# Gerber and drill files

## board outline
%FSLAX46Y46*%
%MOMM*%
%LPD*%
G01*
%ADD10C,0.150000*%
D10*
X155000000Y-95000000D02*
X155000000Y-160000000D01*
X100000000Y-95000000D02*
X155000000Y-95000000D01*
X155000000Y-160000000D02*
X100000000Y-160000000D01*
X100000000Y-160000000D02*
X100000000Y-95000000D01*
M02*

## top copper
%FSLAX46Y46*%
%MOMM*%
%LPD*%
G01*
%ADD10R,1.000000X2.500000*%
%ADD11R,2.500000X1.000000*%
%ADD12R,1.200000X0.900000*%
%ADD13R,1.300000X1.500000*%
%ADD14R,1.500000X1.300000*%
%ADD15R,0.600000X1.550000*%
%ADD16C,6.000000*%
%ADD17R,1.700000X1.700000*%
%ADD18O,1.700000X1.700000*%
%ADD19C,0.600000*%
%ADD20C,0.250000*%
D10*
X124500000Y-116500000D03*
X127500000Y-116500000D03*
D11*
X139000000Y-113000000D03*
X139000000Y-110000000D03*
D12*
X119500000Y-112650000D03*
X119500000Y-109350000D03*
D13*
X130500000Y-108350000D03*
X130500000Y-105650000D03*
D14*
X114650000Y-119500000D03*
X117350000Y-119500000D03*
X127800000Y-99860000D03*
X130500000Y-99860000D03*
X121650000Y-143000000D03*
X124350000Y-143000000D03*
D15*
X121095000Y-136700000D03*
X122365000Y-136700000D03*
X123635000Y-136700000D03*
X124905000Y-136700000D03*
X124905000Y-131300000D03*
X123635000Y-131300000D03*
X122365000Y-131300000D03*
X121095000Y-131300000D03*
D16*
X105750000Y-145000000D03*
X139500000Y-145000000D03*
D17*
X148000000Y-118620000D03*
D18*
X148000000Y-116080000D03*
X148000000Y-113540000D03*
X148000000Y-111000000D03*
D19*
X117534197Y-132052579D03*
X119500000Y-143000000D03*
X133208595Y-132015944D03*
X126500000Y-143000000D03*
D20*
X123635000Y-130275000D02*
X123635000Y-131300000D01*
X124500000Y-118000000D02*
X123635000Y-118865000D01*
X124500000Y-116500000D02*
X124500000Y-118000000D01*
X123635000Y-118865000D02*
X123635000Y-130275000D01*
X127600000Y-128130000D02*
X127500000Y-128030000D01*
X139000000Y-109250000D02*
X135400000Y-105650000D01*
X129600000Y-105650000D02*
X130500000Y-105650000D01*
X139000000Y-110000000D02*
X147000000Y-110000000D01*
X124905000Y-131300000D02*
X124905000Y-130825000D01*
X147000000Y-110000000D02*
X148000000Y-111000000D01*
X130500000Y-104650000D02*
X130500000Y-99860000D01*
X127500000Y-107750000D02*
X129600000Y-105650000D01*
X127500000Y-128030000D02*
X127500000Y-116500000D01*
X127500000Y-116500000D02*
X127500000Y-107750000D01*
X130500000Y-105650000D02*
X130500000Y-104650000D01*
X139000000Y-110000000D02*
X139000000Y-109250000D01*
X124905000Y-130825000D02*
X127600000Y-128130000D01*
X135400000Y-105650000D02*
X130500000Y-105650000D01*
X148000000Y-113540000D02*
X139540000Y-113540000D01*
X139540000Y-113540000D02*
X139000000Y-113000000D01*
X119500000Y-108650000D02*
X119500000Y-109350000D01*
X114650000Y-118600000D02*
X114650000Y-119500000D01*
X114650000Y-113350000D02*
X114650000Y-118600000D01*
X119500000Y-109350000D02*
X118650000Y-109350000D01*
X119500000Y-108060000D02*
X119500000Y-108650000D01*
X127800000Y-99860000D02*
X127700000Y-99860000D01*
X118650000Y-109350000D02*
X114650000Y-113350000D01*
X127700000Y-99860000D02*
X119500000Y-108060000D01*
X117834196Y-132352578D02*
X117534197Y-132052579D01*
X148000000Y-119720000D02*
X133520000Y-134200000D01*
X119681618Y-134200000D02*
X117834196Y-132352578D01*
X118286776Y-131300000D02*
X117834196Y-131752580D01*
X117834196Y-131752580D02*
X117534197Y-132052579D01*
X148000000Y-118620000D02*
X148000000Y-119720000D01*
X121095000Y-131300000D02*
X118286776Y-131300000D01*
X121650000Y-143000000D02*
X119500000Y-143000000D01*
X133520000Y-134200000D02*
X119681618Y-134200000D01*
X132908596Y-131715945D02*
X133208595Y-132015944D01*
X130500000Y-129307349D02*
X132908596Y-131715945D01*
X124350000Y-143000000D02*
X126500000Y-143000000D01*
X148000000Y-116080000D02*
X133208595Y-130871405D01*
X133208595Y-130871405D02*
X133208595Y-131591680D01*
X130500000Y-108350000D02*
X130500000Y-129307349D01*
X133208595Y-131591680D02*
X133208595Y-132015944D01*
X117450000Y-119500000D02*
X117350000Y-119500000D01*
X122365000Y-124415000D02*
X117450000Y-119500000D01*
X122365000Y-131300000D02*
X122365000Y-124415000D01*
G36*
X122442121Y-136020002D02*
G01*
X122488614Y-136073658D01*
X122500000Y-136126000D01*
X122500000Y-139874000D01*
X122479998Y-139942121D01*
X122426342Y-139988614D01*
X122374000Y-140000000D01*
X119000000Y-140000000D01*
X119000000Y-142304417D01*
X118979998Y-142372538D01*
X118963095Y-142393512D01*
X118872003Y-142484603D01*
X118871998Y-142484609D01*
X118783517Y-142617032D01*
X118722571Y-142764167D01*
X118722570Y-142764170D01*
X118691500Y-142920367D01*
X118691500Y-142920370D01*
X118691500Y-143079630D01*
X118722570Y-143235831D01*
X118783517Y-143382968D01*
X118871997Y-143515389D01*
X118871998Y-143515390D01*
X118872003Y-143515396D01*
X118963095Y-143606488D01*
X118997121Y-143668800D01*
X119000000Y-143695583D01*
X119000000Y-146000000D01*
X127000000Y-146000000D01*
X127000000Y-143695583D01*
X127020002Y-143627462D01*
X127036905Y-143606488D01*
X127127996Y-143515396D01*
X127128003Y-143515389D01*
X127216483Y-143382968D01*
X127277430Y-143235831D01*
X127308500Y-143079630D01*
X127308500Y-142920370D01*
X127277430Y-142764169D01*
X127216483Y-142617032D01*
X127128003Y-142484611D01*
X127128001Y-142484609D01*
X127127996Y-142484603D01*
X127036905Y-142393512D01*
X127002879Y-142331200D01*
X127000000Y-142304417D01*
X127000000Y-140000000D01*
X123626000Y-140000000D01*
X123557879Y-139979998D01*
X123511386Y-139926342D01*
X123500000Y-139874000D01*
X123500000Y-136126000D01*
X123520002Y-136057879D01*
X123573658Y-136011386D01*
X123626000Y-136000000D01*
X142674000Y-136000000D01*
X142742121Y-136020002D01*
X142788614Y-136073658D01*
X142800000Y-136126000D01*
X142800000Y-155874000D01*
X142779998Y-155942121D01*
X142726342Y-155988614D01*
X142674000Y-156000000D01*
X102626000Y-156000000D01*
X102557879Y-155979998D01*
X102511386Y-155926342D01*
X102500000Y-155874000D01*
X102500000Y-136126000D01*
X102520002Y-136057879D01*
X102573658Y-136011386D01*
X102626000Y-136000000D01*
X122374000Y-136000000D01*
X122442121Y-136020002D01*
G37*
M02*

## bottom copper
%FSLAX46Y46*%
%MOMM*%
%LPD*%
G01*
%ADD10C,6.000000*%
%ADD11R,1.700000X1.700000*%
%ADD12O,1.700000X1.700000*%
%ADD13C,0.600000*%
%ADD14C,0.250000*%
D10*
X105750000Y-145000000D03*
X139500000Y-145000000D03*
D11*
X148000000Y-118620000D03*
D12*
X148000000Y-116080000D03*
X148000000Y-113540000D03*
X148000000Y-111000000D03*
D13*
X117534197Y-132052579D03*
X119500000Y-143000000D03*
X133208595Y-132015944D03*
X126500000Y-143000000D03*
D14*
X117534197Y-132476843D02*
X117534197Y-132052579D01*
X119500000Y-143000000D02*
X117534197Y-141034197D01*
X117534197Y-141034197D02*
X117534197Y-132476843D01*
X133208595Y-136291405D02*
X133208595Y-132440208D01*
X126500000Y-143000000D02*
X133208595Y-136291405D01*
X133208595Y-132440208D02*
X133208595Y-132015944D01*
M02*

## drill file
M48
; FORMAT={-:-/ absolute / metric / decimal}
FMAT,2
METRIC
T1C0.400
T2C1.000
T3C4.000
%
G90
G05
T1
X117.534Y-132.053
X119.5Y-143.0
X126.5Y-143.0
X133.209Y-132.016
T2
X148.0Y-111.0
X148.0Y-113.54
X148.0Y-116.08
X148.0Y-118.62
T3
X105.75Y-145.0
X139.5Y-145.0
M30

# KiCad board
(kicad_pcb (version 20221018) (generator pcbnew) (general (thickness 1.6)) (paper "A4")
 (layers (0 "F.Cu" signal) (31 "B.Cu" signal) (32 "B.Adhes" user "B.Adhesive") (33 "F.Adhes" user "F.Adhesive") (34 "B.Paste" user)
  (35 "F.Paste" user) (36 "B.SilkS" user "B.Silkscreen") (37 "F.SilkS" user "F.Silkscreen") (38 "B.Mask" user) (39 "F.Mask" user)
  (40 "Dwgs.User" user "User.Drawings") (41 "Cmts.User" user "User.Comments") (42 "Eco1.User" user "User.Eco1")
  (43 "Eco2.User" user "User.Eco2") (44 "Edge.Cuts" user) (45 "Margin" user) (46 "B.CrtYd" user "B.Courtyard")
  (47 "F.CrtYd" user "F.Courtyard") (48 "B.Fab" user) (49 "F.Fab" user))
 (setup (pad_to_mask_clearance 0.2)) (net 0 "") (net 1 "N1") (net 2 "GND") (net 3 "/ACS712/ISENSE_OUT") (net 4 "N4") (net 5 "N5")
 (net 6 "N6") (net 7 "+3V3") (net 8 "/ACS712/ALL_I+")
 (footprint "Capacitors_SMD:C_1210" (layer "F.Cu") (at 126 116.5)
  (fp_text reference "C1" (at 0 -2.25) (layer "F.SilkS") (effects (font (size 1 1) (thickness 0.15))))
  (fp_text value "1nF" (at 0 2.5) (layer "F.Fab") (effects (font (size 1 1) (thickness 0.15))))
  (pad "1" smd rect (at -1.5 0) (size 1 2.5) (layers "F.Cu" "F.Paste" "F.Mask") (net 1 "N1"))
  (pad "2" smd rect (at 1.5 0) (size 1 2.5) (layers "F.Cu" "F.Paste" "F.Mask") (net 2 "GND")))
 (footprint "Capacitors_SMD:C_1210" (layer "F.Cu") (at 139 111.5 90)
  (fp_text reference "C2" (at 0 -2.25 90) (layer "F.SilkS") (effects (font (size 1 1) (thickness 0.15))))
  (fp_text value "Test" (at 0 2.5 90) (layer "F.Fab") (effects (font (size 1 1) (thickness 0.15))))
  (pad "1" smd rect (at -1.5 0 90) (size 1 2.5) (layers "F.Cu" "F.Paste" "F.Mask") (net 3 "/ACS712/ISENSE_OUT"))
  (pad "2" smd rect (at 1.5 0 90) (size 1 2.5) (layers "F.Cu" "F.Paste" "F.Mask") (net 2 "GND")))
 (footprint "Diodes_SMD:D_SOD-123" (layer "F.Cu") (at 119.5 111 90)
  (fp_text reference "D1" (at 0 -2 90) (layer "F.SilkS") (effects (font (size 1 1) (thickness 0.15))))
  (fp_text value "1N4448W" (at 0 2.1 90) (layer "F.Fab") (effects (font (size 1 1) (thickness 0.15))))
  (pad "1" smd rect (at -1.65 0 90) (size 0.9 1.2) (layers "F.Cu" "F.Paste" "F.Mask") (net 3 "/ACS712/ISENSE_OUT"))
  (pad "2" smd rect (at 1.65 0 90) (size 0.9 1.2) (layers "F.Cu" "F.Paste" "F.Mask") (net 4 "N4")))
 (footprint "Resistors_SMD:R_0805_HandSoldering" (layer "F.Cu") (at 130.5 107 90)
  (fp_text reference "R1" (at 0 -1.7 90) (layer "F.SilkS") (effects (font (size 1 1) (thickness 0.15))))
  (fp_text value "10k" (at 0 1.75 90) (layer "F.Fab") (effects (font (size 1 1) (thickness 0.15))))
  (pad "1" smd rect (at -1.35 0 90) (size 1.5 1.3) (layers "F.Cu" "F.Paste" "F.Mask") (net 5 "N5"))
  (pad "2" smd rect (at 1.35 0 90) (size 1.5 1.3) (layers "F.Cu" "F.Paste" "F.Mask") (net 2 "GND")))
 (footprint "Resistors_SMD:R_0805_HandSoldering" (layer "F.Cu") (at 116 119.5)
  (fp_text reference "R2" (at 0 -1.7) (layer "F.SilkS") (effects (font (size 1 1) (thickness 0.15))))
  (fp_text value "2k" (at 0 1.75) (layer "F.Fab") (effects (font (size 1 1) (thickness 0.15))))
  (pad "1" smd rect (at -1.35 0) (size 1.5 1.3) (layers "F.Cu" "F.Paste" "F.Mask") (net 4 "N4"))
  (pad "2" smd rect (at 1.35 0) (size 1.5 1.3) (layers "F.Cu" "F.Paste" "F.Mask") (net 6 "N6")))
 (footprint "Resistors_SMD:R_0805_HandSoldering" (layer "F.Cu") (at 129.15 99.86)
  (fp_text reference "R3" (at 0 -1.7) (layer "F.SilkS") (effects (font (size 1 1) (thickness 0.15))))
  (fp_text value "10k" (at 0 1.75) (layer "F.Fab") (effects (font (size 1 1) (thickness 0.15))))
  (pad "1" smd rect (at -1.35 0) (size 1.5 1.3) (layers "F.Cu" "F.Paste" "F.Mask") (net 4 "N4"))
  (pad "2" smd rect (at 1.35 0) (size 1.5 1.3) (layers "F.Cu" "F.Paste" "F.Mask") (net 2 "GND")))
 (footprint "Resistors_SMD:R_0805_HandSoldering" (layer "F.Cu") (at 123 143)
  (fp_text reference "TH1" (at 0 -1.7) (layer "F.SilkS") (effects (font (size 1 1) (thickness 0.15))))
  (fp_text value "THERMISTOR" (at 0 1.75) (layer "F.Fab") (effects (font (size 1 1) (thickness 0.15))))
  (pad "1" smd rect (at -1.35 0) (size 1.5 1.3) (layers "F.Cu" "F.Paste" "F.Mask") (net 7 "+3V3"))
  (pad "2" smd rect (at 1.35 0) (size 1.5 1.3) (layers "F.Cu" "F.Paste" "F.Mask") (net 5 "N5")))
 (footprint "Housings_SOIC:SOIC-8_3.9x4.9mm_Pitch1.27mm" (layer "F.Cu") (at 123 134 90)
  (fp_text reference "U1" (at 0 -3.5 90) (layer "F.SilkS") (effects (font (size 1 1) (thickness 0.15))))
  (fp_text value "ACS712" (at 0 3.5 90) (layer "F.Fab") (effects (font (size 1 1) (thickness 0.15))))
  (pad "1" smd rect (at -2.7 -1.905 90) (size 1.55 0.6) (layers "F.Cu" "F.Paste" "F.Mask") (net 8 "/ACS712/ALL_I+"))
  (pad "2" smd rect (at -2.7 -0.635 90) (size 1.55 0.6) (layers "F.Cu" "F.Paste" "F.Mask") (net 8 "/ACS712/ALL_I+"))
  (pad "3" smd rect (at -2.7 0.635 90) (size 1.55 0.6) (layers "F.Cu" "F.Paste" "F.Mask") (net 8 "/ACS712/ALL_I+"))
  (pad "4" smd rect (at -2.7 1.905 90) (size 1.55 0.6) (layers "F.Cu" "F.Paste" "F.Mask") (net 8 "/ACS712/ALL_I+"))
  (pad "5" smd rect (at 2.7 1.905 90) (size 1.55 0.6) (layers "F.Cu" "F.Paste" "F.Mask") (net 2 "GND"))
  (pad "6" smd rect (at 2.7 0.635 90) (size 1.55 0.6) (layers "F.Cu" "F.Paste" "F.Mask") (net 1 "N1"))
  (pad "7" smd rect (at 2.7 -0.635 90) (size 1.55 0.6) (layers "F.Cu" "F.Paste" "F.Mask") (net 6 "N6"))
  (pad "8" smd rect (at 2.7 -1.905 90) (size 1.55 0.6) (layers "F.Cu" "F.Paste" "F.Mask") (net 7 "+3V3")))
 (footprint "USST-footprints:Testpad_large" (layer "F.Cu") (at 105.75 145)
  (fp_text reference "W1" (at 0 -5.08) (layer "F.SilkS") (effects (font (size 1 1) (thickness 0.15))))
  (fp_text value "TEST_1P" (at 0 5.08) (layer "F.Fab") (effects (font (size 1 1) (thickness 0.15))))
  (pad "1" thru_hole circle (at 0 0) (size 6 6) (drill 4) (layers "*.Cu" "*.Mask") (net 8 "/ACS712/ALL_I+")))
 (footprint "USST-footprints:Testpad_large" (layer "F.Cu") (at 139.5 145)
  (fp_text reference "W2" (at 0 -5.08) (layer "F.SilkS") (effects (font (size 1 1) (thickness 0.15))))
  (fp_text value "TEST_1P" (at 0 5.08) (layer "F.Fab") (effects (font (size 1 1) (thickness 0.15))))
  (pad "1" thru_hole circle (at 0 0) (size 6 6) (drill 4) (layers "*.Cu" "*.Mask") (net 8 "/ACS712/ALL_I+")))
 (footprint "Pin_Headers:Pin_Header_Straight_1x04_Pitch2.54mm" (layer "B.Cu") (at 148 118.62)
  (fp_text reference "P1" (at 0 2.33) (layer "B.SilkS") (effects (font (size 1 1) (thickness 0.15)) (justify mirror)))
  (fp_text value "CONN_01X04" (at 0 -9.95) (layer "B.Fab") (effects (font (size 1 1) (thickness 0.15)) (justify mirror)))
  (pad "1" thru_hole rect (at 0 0) (size 1.7 1.7) (drill 1) (layers "*.Cu" "*.Mask") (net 7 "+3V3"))
  (pad "2" thru_hole oval (at 0 -2.54) (size 1.7 1.7) (drill 1) (layers "*.Cu" "*.Mask") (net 5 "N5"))
  (pad "3" thru_hole oval (at 0 -5.08) (size 1.7 1.7) (drill 1) (layers "*.Cu" "*.Mask") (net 3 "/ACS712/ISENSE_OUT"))
  (pad "4" thru_hole oval (at 0 -7.62) (size 1.7 1.7) (drill 1) (layers "*.Cu" "*.Mask") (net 2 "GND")))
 (gr_line (start 155 95) (end 155 160) (stroke (width 0.15) (type solid)) (layer "Edge.Cuts"))
 (gr_line (start 100 95) (end 155 95) (stroke (width 0.15) (type solid)) (layer "Edge.Cuts"))
 (gr_line (start 155 160) (end 100 160) (stroke (width 0.15) (type solid)) (layer "Edge.Cuts"))
 (gr_line (start 100 160) (end 100 95) (stroke (width 0.15) (type solid)) (layer "Edge.Cuts"))
 (segment (start 123.635 130.275) (end 123.635 131.3) (width 0.25) (layer "F.Cu") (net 1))
 (segment (start 124.5 118) (end 123.635 118.865) (width 0.25) (layer "F.Cu") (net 1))
 (segment (start 124.5 116.5) (end 124.5 118) (width 0.25) (layer "F.Cu") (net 1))
 (segment (start 123.635 118.865) (end 123.635 130.275) (width 0.25) (layer "F.Cu") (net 1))
 (segment (start 127.6 128.13) (end 127.5 128.03) (width 0.25) (layer "F.Cu") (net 2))
 (segment (start 139 109.25) (end 135.4 105.65) (width 0.25) (layer "F.Cu") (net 2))
 (segment (start 129.6 105.65) (end 130.5 105.65) (width 0.25) (layer "F.Cu") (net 2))
 (segment (start 139 110) (end 147 110) (width 0.25) (layer "F.Cu") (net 2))
 (segment (start 124.905 131.3) (end 124.905 130.825) (width 0.25) (layer "F.Cu") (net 2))
 (segment (start 147 110) (end 148 111) (width 0.25) (layer "F.Cu") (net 2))
 (segment (start 130.5 104.65) (end 130.5 99.86) (width 0.25) (layer "F.Cu") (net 2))
 (segment (start 127.5 107.75) (end 129.6 105.65) (width 0.25) (layer "F.Cu") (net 2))
 (segment (start 127.5 128.03) (end 127.5 116.5) (width 0.25) (layer "F.Cu") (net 2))
 (segment (start 127.5 116.5) (end 127.5 107.75) (width 0.25) (layer "F.Cu") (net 2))
 (segment (start 130.5 105.65) (end 130.5 104.65) (width 0.25) (layer "F.Cu") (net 2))
 (segment (start 139 110) (end 139 109.25) (width 0.25) (layer "F.Cu") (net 2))
 (segment (start 124.905 130.825) (end 127.6 128.13) (width 0.25) (layer "F.Cu") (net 2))
 (segment (start 135.4 105.65) (end 130.5 105.65) (width 0.25) (layer "F.Cu") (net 2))
 (segment (start 148 113.54) (end 139.54 113.54) (width 0.25) (layer "F.Cu") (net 3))
 (segment (start 139.54 113.54) (end 139 113) (width 0.25) (layer "F.Cu") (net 3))
 (segment (start 119.5 108.65) (end 119.5 109.35) (width 0.25) (layer "F.Cu") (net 4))
 (segment (start 114.65 118.6) (end 114.65 119.5) (width 0.25) (layer "F.Cu") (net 4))
 (segment (start 114.65 113.35) (end 114.65 118.6) (width 0.25) (layer "F.Cu") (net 4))
 (segment (start 119.5 109.35) (end 118.65 109.35) (width 0.25) (layer "F.Cu") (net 4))
 (segment (start 119.5 108.06) (end 119.5 108.65) (width 0.25) (layer "F.Cu") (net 4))
 (segment (start 127.8 99.86) (end 127.7 99.86) (width 0.25) (layer "F.Cu") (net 4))
 (segment (start 118.65 109.35) (end 114.65 113.35) (width 0.25) (layer "F.Cu") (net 4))
 (segment (start 127.7 99.86) (end 119.5 108.06) (width 0.25) (layer "F.Cu") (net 4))
 (segment (start 117.834196 132.352578) (end 117.534197 132.052579) (width 0.25) (layer "F.Cu") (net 7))
 (segment (start 148 119.72) (end 133.52 134.2) (width 0.25) (layer "F.Cu") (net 7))
 (segment (start 119.681618 134.2) (end 117.834196 132.352578) (width 0.25) (layer "F.Cu") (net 7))
 (segment (start 118.286776 131.3) (end 117.834196 131.75258) (width 0.25) (layer "F.Cu") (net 7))
 (segment (start 117.834196 131.75258) (end 117.534197 132.052579) (width 0.25) (layer "F.Cu") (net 7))
 (segment (start 148 118.62) (end 148 119.72) (width 0.25) (layer "F.Cu") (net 7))
 (segment (start 121.095 131.3) (end 118.286776 131.3) (width 0.25) (layer "F.Cu") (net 7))
 (segment (start 121.65 143) (end 119.5 143) (width 0.25) (layer "F.Cu") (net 7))
 (segment (start 133.52 134.2) (end 119.681618 134.2) (width 0.25) (layer "F.Cu") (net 7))
 (via (at 117.534197 132.052579) (size 0.6) (drill 0.4) (layers "F.Cu" "B.Cu") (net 7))
 (via (at 119.5 143) (size 0.6) (drill 0.4) (layers "F.Cu" "B.Cu") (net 7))
 (segment (start 117.534197 132.476843) (end 117.534197 132.052579) (width 0.25) (layer "B.Cu") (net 7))
 (segment (start 119.5 143) (end 117.534197 141.034197) (width 0.25) (layer "B.Cu") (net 7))
 (segment (start 117.534197 141.034197) (end 117.534197 132.476843) (width 0.25) (layer "B.Cu") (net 7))
 (segment (start 132.908596 131.715945) (end 133.208595 132.015944) (width 0.25) (layer "F.Cu") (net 5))
 (segment (start 130.5 129.307349) (end 132.908596 131.715945) (width 0.25) (layer "F.Cu") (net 5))
 (segment (start 124.35 143) (end 126.5 143) (width 0.25) (layer "F.Cu") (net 5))
 (segment (start 148 116.08) (end 133.208595 130.871405) (width 0.25) (layer "F.Cu") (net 5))
 (segment (start 133.208595 130.871405) (end 133.208595 131.59168) (width 0.25) (layer "F.Cu") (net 5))
 (segment (start 130.5 108.35) (end 130.5 129.307349) (width 0.25) (layer "F.Cu") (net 5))
 (segment (start 133.208595 131.59168) (end 133.208595 132.015944) (width 0.25) (layer "F.Cu") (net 5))
 (via (at 133.208595 132.015944) (size 0.6) (drill 0.4) (layers "F.Cu" "B.Cu") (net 5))
 (via (at 126.5 143) (size 0.6) (drill 0.4) (layers "F.Cu" "B.Cu") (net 5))
 (segment (start 133.208595 136.291405) (end 133.208595 132.440208) (width 0.25) (layer "B.Cu") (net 5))
 (segment (start 126.5 143) (end 133.208595 136.291405) (width 0.25) (layer "B.Cu") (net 5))
 (segment (start 133.208595 132.440208) (end 133.208595 132.015944) (width 0.25) (layer "B.Cu") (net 5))
 (segment (start 117.45 119.5) (end 117.35 119.5) (width 0.25) (layer "F.Cu") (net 6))
 (segment (start 122.365 124.415) (end 117.45 119.5) (width 0.25) (layer "F.Cu") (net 6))
 (segment (start 122.365 131.3) (end 122.365 124.415) (width 0.25) (layer "F.Cu") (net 6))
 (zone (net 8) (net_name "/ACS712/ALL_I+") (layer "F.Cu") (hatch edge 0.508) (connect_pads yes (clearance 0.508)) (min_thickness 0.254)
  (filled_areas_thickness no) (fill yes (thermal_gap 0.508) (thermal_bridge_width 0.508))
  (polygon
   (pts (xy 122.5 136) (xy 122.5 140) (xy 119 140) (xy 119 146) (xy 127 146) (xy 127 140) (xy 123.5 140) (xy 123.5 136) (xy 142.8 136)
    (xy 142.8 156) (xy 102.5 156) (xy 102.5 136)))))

